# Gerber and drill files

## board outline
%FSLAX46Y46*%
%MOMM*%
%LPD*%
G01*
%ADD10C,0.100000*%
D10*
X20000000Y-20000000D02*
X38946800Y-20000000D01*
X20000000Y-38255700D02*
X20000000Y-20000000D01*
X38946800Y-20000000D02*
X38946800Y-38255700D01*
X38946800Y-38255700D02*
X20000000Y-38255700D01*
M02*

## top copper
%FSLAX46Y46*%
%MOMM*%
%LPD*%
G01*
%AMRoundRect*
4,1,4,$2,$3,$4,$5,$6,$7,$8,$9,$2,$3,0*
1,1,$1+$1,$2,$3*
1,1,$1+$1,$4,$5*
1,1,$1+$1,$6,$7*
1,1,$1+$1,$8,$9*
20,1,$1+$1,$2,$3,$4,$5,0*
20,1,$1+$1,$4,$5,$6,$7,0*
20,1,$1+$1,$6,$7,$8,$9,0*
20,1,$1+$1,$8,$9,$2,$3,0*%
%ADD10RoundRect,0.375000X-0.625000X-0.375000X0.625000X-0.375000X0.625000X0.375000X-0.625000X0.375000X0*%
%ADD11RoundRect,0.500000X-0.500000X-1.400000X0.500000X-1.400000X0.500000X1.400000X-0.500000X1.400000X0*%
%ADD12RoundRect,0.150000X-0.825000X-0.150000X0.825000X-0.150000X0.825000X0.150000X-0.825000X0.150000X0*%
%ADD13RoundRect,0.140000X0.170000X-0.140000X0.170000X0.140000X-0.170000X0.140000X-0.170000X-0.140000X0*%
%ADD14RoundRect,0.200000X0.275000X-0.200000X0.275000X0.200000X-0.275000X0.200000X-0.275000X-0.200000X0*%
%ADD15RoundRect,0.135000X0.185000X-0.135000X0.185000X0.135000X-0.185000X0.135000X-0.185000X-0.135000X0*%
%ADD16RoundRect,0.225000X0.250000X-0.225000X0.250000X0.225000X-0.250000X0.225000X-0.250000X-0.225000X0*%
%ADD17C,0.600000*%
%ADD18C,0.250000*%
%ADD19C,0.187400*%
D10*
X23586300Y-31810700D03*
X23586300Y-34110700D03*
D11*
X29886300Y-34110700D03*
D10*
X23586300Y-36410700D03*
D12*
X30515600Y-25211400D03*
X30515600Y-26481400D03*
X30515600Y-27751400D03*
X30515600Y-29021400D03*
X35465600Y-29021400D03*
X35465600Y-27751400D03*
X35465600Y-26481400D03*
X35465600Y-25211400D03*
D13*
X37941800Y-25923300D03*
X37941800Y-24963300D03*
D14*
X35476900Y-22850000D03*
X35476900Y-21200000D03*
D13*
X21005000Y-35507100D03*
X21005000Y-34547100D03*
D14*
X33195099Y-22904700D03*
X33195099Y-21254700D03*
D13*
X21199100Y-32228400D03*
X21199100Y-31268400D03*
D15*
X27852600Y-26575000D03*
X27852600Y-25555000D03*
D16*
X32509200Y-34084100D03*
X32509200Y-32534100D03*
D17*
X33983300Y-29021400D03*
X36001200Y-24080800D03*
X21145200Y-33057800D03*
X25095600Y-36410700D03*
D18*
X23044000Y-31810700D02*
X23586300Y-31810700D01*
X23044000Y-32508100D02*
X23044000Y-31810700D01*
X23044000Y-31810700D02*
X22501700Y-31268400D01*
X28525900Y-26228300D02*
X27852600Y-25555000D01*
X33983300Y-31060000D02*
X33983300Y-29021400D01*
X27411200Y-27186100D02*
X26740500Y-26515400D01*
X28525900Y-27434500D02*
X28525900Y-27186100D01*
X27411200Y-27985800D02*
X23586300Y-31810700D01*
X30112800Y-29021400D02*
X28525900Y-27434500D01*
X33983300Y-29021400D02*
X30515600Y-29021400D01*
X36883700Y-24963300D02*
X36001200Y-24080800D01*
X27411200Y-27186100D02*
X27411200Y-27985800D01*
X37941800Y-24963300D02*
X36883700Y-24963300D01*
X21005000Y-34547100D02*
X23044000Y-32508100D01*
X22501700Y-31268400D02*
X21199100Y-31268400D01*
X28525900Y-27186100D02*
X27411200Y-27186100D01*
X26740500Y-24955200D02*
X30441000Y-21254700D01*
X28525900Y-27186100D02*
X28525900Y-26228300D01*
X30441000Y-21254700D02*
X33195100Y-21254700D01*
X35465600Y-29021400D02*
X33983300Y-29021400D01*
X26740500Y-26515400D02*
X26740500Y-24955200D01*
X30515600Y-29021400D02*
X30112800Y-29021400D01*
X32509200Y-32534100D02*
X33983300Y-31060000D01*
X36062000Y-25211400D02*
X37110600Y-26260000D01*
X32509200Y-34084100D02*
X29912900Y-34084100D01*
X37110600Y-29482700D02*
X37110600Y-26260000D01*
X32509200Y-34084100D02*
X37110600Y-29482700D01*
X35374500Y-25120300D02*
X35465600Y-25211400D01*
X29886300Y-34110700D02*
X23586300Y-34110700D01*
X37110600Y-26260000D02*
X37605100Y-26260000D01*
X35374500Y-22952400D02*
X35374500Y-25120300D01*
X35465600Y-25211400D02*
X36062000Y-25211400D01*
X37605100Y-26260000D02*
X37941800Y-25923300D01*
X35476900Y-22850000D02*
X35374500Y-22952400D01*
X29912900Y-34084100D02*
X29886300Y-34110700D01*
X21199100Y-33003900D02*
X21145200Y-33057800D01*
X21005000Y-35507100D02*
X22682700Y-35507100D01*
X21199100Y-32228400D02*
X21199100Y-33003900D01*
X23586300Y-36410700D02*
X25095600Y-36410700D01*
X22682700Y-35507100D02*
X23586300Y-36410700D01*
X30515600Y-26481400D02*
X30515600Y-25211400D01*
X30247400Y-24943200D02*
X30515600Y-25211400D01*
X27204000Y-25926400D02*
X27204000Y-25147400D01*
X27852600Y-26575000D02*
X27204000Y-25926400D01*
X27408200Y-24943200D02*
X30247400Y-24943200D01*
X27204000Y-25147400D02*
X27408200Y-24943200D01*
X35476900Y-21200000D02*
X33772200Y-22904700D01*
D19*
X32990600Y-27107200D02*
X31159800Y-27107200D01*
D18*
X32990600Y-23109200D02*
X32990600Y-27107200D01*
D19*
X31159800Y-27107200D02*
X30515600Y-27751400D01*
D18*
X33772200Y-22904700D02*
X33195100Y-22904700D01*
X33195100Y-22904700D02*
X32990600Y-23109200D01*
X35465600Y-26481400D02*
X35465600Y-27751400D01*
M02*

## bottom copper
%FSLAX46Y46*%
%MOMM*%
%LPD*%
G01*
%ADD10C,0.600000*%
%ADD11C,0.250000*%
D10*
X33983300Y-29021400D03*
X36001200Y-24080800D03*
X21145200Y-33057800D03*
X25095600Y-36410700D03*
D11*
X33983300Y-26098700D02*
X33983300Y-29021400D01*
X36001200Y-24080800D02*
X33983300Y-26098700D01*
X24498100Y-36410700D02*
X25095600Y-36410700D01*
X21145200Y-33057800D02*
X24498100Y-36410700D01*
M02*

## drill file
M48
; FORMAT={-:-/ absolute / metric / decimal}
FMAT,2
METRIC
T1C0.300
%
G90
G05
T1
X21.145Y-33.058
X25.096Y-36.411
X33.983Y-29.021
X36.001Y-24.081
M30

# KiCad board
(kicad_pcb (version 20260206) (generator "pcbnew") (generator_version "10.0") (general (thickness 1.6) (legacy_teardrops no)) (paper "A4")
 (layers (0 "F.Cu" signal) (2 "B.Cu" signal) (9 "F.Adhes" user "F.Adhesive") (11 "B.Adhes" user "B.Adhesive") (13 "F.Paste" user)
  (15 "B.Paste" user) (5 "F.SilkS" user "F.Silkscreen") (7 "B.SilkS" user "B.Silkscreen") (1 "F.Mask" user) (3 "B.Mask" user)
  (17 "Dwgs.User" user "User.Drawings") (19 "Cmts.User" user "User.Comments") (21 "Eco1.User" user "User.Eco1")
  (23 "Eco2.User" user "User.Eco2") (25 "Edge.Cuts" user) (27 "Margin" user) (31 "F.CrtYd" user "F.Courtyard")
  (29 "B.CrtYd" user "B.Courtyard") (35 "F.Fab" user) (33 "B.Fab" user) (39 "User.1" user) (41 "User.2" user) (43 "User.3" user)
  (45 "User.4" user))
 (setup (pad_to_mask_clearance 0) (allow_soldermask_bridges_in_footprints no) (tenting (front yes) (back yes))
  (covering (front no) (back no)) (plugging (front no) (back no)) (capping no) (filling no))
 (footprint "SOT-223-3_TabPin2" (layer "F.Cu") (at 26.7363 34.1107)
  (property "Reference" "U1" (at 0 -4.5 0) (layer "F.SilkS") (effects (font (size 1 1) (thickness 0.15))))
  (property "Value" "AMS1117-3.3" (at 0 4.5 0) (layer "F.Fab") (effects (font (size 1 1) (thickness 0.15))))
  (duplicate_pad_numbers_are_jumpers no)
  (pad "1" smd roundrect (at -3.15 -2.3) (size 2 1.5) (layers "F.Cu" "F.Mask" "F.Paste") (roundrect_rratio 0.25) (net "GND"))
  (pad "2" smd roundrect (at -3.15 0) (size 2 1.5) (layers "F.Cu" "F.Mask" "F.Paste") (roundrect_rratio 0.25) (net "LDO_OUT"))
  (pad "2" smd roundrect (at 3.15 0) (size 2 3.8) (layers "F.Cu" "F.Mask" "F.Paste") (roundrect_rratio 0.25) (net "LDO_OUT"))
  (pad "3" smd roundrect (at -3.15 2.3) (size 2 1.5) (layers "F.Cu" "F.Mask" "F.Paste") (roundrect_rratio 0.25) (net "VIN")))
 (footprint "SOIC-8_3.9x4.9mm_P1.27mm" (layer "F.Cu") (at 32.9906 27.1164)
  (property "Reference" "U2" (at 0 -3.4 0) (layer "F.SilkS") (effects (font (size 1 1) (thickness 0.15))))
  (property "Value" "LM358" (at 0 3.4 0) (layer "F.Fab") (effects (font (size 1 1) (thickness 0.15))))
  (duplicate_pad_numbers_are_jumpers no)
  (pad "1" smd roundrect (at -2.475 -1.905) (size 1.95 0.6) (layers "F.Cu" "F.Mask" "F.Paste") (roundrect_rratio 0.25) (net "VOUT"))
  (pad "2" smd roundrect (at -2.475 -0.635) (size 1.95 0.6) (layers "F.Cu" "F.Mask" "F.Paste") (roundrect_rratio 0.25) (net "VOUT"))
  (pad "3" smd roundrect (at -2.475 0.635) (size 1.95 0.6) (layers "F.Cu" "F.Mask" "F.Paste") (roundrect_rratio 0.25) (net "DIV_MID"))
  (pad "4" smd roundrect (at -2.475 1.905) (size 1.95 0.6) (layers "F.Cu" "F.Mask" "F.Paste") (roundrect_rratio 0.25) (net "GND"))
  (pad "5" smd roundrect (at 2.475 1.905) (size 1.95 0.6) (layers "F.Cu" "F.Mask" "F.Paste") (roundrect_rratio 0.25) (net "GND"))
  (pad "6" smd roundrect (at 2.475 0.635) (size 1.95 0.6) (layers "F.Cu" "F.Mask" "F.Paste") (roundrect_rratio 0.25) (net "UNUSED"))
  (pad "7" smd roundrect (at 2.475 -0.635) (size 1.95 0.6) (layers "F.Cu" "F.Mask" "F.Paste") (roundrect_rratio 0.25) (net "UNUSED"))
  (pad "8" smd roundrect (at 2.475 -1.905) (size 1.95 0.6) (layers "F.Cu" "F.Mask" "F.Paste") (roundrect_rratio 0.25) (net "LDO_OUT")))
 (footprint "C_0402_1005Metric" (layer "F.Cu") (at 37.9418 25.4433 90)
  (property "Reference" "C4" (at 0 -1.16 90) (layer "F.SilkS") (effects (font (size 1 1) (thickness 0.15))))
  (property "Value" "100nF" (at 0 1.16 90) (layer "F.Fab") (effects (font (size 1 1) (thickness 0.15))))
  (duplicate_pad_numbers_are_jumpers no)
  (pad "1" smd roundrect (at -0.48 0 90) (size 0.56 0.62) (layers "F.Cu" "F.Mask" "F.Paste") (roundrect_rratio 0.25) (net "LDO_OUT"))
  (pad "2" smd roundrect (at 0.48 0 90) (size 0.56 0.62) (layers "F.Cu" "F.Mask" "F.Paste") (roundrect_rratio 0.25) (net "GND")))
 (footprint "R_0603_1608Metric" (layer "F.Cu") (at 35.4769 22.025 90)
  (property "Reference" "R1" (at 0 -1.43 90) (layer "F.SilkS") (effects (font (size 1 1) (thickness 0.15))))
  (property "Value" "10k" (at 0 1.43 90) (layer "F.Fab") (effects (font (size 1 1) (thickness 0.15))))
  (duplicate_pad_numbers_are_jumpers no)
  (pad "1" smd roundrect (at -0.825 0 90) (size 0.8 0.95) (layers "F.Cu" "F.Mask" "F.Paste") (roundrect_rratio 0.25) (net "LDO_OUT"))
  (pad "2" smd roundrect (at 0.825 0 90) (size 0.8 0.95) (layers "F.Cu" "F.Mask" "F.Paste") (roundrect_rratio 0.25) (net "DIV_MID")))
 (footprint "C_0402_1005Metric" (layer "F.Cu") (at 21.005 35.0271 90)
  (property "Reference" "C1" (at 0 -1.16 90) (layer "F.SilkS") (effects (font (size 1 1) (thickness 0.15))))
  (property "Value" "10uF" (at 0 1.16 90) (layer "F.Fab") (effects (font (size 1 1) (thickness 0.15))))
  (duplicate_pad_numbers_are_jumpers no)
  (pad "1" smd roundrect (at -0.48 0 90) (size 0.56 0.62) (layers "F.Cu" "F.Mask" "F.Paste") (roundrect_rratio 0.25) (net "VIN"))
  (pad "2" smd roundrect (at 0.48 0 90) (size 0.56 0.62) (layers "F.Cu" "F.Mask" "F.Paste") (roundrect_rratio 0.25) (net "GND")))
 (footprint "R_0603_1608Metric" (layer "F.Cu") (at 33.195099 22.0797 90)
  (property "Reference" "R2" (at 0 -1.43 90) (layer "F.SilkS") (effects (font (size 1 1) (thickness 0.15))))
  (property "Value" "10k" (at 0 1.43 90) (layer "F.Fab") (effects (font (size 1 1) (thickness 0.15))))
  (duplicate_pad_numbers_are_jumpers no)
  (pad "1" smd roundrect (at -0.825 0 90) (size 0.8 0.95) (layers "F.Cu" "F.Mask" "F.Paste") (roundrect_rratio 0.25) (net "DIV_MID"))
  (pad "2" smd roundrect (at 0.825 0 90) (size 0.8 0.95) (layers "F.Cu" "F.Mask" "F.Paste") (roundrect_rratio 0.25) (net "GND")))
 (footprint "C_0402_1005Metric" (layer "F.Cu") (at 21.1991 31.7484 90)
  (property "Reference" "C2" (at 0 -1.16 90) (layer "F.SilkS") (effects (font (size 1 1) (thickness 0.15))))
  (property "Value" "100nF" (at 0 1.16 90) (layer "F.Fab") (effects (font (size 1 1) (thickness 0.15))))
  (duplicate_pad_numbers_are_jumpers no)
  (pad "1" smd roundrect (at -0.48 0 90) (size 0.56 0.62) (layers "F.Cu" "F.Mask" "F.Paste") (roundrect_rratio 0.25) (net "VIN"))
  (pad "2" smd roundrect (at 0.48 0 90) (size 0.56 0.62) (layers "F.Cu" "F.Mask" "F.Paste") (roundrect_rratio 0.25) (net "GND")))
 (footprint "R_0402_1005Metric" (layer "F.Cu") (at 27.8526 26.065 90)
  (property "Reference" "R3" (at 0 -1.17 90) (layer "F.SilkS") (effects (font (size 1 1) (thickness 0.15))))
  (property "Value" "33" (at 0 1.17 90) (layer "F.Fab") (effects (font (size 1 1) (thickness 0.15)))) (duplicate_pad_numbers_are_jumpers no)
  (pad "1" smd roundrect (at -0.51 0 90) (size 0.54 0.64) (layers "F.Cu" "F.Mask" "F.Paste") (roundrect_rratio 0.25) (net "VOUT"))
  (pad "2" smd roundrect (at 0.51 0 90) (size 0.54 0.64) (layers "F.Cu" "F.Mask" "F.Paste") (roundrect_rratio 0.25) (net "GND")))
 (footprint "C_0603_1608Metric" (layer "F.Cu") (at 32.5092 33.3091 90)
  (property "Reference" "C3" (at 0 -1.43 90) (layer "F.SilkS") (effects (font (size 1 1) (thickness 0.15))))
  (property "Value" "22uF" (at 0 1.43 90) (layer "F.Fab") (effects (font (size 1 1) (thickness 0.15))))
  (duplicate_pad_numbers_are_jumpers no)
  (pad "1" smd roundrect (at -0.775 0 90) (size 0.9 0.95) (layers "F.Cu" "F.Mask" "F.Paste") (roundrect_rratio 0.25) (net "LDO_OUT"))
  (pad "2" smd roundrect (at 0.775 0 90) (size 0.9 0.95) (layers "F.Cu" "F.Mask" "F.Paste") (roundrect_rratio 0.25) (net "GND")))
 (gr_line (start 20 20) (end 38.9468 20) (stroke (width 0.1) (type default)) (layer "Edge.Cuts"))
 (gr_line (start 20 38.2557) (end 20 20) (stroke (width 0.1) (type default)) (layer "Edge.Cuts"))
 (gr_line (start 38.9468 20) (end 38.9468 38.2557) (stroke (width 0.1) (type default)) (layer "Edge.Cuts"))
 (gr_line (start 38.9468 38.2557) (end 20 38.2557) (stroke (width 0.1) (type default)) (layer "Edge.Cuts"))
 (segment (start 23.044 31.8107) (end 23.5863 31.8107) (width 0.25) (layer "F.Cu") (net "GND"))
 (segment (start 23.044 32.5081) (end 23.044 31.8107) (width 0.25) (layer "F.Cu") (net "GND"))
 (segment (start 23.044 31.8107) (end 22.5017 31.2684) (width 0.25) (layer "F.Cu") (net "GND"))
 (segment (start 28.5259 26.2283) (end 27.8526 25.555) (width 0.25) (layer "F.Cu") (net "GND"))
 (segment (start 33.9833 31.06) (end 33.9833 29.0214) (width 0.25) (layer "F.Cu") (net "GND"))
 (segment (start 27.4112 27.1861) (end 26.7405 26.5154) (width 0.25) (layer "F.Cu") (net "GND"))
 (segment (start 28.5259 27.4345) (end 28.5259 27.1861) (width 0.25) (layer "F.Cu") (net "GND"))
 (segment (start 27.4112 27.9858) (end 23.5863 31.8107) (width 0.25) (layer "F.Cu") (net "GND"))
 (segment (start 30.1128 29.0214) (end 28.5259 27.4345) (width 0.25) (layer "F.Cu") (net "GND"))
 (segment (start 33.9833 29.0214) (end 30.5156 29.0214) (width 0.25) (layer "F.Cu") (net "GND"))
 (segment (start 36.8837 24.9633) (end 36.0012 24.0808) (width 0.25) (layer "F.Cu") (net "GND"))
 (segment (start 27.4112 27.1861) (end 27.4112 27.9858) (width 0.25) (layer "F.Cu") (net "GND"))
 (segment (start 37.9418 24.9633) (end 36.8837 24.9633) (width 0.25) (layer "F.Cu") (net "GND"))
 (segment (start 21.005 34.5471) (end 23.044 32.5081) (width 0.25) (layer "F.Cu") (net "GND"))
 (segment (start 22.5017 31.2684) (end 21.1991 31.2684) (width 0.25) (layer "F.Cu") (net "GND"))
 (segment (start 28.5259 27.1861) (end 27.4112 27.1861) (width 0.25) (layer "F.Cu") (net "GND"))
 (segment (start 26.7405 24.9552) (end 30.441 21.2547) (width 0.25) (layer "F.Cu") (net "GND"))
 (segment (start 28.5259 27.1861) (end 28.5259 26.2283) (width 0.25) (layer "F.Cu") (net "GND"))
 (segment (start 30.441 21.2547) (end 33.1951 21.2547) (width 0.25) (layer "F.Cu") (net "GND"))
 (segment (start 35.4656 29.0214) (end 33.9833 29.0214) (width 0.25) (layer "F.Cu") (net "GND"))
 (segment (start 26.7405 26.5154) (end 26.7405 24.9552) (width 0.25) (layer "F.Cu") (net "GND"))
 (segment (start 30.5156 29.0214) (end 30.1128 29.0214) (width 0.25) (layer "F.Cu") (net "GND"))
 (segment (start 32.5092 32.5341) (end 33.9833 31.06) (width 0.25) (layer "F.Cu") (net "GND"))
 (via (at 33.9833 29.0214) (size 0.6) (drill 0.3) (layers "F.Cu" "B.Cu") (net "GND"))
 (via (at 36.0012 24.0808) (size 0.6) (drill 0.3) (layers "F.Cu" "B.Cu") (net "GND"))
 (segment (start 33.9833 26.0987) (end 33.9833 29.0214) (width 0.25) (layer "B.Cu") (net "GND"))
 (segment (start 36.0012 24.0808) (end 33.9833 26.0987) (width 0.25) (layer "B.Cu") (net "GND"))
 (segment (start 36.062 25.2114) (end 37.1106 26.26) (width 0.25) (layer "F.Cu") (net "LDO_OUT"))
 (segment (start 32.5092 34.0841) (end 29.9129 34.0841) (width 0.25) (layer "F.Cu") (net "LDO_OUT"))
 (segment (start 37.1106 29.4827) (end 37.1106 26.26) (width 0.25) (layer "F.Cu") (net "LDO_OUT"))
 (segment (start 32.5092 34.0841) (end 37.1106 29.4827) (width 0.25) (layer "F.Cu") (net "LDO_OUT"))
 (segment (start 35.3745 25.1203) (end 35.4656 25.2114) (width 0.25) (layer "F.Cu") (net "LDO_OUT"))
 (segment (start 29.8863 34.1107) (end 23.5863 34.1107) (width 0.25) (layer "F.Cu") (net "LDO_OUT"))
 (segment (start 37.1106 26.26) (end 37.6051 26.26) (width 0.25) (layer "F.Cu") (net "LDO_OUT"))
 (segment (start 35.3745 22.9524) (end 35.3745 25.1203) (width 0.25) (layer "F.Cu") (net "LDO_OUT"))
 (segment (start 35.4656 25.2114) (end 36.062 25.2114) (width 0.25) (layer "F.Cu") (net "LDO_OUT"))
 (segment (start 37.6051 26.26) (end 37.9418 25.9233) (width 0.25) (layer "F.Cu") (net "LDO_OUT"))
 (segment (start 35.4769 22.85) (end 35.3745 22.9524) (width 0.25) (layer "F.Cu") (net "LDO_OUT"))
 (segment (start 29.9129 34.0841) (end 29.8863 34.1107) (width 0.25) (layer "F.Cu") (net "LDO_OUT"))
 (segment (start 21.1991 33.0039) (end 21.1452 33.0578) (width 0.25) (layer "F.Cu") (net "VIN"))
 (segment (start 21.005 35.5071) (end 22.6827 35.5071) (width 0.25) (layer "F.Cu") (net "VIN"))
 (segment (start 21.1991 32.2284) (end 21.1991 33.0039) (width 0.25) (layer "F.Cu") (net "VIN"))
 (segment (start 23.5863 36.4107) (end 25.0956 36.4107) (width 0.25) (layer "F.Cu") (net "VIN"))
 (segment (start 22.6827 35.5071) (end 23.5863 36.4107) (width 0.25) (layer "F.Cu") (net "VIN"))
 (via (at 21.1452 33.0578) (size 0.6) (drill 0.3) (layers "F.Cu" "B.Cu") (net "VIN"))
 (via (at 25.0956 36.4107) (size 0.6) (drill 0.3) (layers "F.Cu" "B.Cu") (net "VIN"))
 (segment (start 24.4981 36.4107) (end 25.0956 36.4107) (width 0.25) (layer "B.Cu") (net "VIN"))
 (segment (start 21.1452 33.0578) (end 24.4981 36.4107) (width 0.25) (layer "B.Cu") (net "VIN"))
 (segment (start 30.5156 26.4814) (end 30.5156 25.2114) (width 0.25) (layer "F.Cu") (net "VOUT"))
 (segment (start 30.2474 24.9432) (end 30.5156 25.2114) (width 0.25) (layer "F.Cu") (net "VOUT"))
 (segment (start 27.204 25.9264) (end 27.204 25.1474) (width 0.25) (layer "F.Cu") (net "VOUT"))
 (segment (start 27.8526 26.575) (end 27.204 25.9264) (width 0.25) (layer "F.Cu") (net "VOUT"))
 (segment (start 27.4082 24.9432) (end 30.2474 24.9432) (width 0.25) (layer "F.Cu") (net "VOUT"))
 (segment (start 27.204 25.1474) (end 27.4082 24.9432) (width 0.25) (layer "F.Cu") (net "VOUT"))
 (segment (start 35.4769 21.2) (end 33.7722 22.9047) (width 0.25) (layer "F.Cu") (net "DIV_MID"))
 (segment (start 32.9906 27.1072) (end 31.1598 27.1072) (width 0.1874) (layer "F.Cu") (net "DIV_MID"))
 (segment (start 32.9906 23.1092) (end 32.9906 27.1072) (width 0.25) (layer "F.Cu") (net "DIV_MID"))
 (segment (start 31.1598 27.1072) (end 30.5156 27.7514) (width 0.1874) (layer "F.Cu") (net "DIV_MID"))
 (segment (start 33.7722 22.9047) (end 33.1951 22.9047) (width 0.25) (layer "F.Cu") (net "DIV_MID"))
 (segment (start 33.1951 22.9047) (end 32.9906 23.1092) (width 0.25) (layer "F.Cu") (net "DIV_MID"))
 (segment (start 35.4656 26.4814) (end 35.4656 27.7514) (width 0.25) (layer "F.Cu") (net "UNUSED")))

